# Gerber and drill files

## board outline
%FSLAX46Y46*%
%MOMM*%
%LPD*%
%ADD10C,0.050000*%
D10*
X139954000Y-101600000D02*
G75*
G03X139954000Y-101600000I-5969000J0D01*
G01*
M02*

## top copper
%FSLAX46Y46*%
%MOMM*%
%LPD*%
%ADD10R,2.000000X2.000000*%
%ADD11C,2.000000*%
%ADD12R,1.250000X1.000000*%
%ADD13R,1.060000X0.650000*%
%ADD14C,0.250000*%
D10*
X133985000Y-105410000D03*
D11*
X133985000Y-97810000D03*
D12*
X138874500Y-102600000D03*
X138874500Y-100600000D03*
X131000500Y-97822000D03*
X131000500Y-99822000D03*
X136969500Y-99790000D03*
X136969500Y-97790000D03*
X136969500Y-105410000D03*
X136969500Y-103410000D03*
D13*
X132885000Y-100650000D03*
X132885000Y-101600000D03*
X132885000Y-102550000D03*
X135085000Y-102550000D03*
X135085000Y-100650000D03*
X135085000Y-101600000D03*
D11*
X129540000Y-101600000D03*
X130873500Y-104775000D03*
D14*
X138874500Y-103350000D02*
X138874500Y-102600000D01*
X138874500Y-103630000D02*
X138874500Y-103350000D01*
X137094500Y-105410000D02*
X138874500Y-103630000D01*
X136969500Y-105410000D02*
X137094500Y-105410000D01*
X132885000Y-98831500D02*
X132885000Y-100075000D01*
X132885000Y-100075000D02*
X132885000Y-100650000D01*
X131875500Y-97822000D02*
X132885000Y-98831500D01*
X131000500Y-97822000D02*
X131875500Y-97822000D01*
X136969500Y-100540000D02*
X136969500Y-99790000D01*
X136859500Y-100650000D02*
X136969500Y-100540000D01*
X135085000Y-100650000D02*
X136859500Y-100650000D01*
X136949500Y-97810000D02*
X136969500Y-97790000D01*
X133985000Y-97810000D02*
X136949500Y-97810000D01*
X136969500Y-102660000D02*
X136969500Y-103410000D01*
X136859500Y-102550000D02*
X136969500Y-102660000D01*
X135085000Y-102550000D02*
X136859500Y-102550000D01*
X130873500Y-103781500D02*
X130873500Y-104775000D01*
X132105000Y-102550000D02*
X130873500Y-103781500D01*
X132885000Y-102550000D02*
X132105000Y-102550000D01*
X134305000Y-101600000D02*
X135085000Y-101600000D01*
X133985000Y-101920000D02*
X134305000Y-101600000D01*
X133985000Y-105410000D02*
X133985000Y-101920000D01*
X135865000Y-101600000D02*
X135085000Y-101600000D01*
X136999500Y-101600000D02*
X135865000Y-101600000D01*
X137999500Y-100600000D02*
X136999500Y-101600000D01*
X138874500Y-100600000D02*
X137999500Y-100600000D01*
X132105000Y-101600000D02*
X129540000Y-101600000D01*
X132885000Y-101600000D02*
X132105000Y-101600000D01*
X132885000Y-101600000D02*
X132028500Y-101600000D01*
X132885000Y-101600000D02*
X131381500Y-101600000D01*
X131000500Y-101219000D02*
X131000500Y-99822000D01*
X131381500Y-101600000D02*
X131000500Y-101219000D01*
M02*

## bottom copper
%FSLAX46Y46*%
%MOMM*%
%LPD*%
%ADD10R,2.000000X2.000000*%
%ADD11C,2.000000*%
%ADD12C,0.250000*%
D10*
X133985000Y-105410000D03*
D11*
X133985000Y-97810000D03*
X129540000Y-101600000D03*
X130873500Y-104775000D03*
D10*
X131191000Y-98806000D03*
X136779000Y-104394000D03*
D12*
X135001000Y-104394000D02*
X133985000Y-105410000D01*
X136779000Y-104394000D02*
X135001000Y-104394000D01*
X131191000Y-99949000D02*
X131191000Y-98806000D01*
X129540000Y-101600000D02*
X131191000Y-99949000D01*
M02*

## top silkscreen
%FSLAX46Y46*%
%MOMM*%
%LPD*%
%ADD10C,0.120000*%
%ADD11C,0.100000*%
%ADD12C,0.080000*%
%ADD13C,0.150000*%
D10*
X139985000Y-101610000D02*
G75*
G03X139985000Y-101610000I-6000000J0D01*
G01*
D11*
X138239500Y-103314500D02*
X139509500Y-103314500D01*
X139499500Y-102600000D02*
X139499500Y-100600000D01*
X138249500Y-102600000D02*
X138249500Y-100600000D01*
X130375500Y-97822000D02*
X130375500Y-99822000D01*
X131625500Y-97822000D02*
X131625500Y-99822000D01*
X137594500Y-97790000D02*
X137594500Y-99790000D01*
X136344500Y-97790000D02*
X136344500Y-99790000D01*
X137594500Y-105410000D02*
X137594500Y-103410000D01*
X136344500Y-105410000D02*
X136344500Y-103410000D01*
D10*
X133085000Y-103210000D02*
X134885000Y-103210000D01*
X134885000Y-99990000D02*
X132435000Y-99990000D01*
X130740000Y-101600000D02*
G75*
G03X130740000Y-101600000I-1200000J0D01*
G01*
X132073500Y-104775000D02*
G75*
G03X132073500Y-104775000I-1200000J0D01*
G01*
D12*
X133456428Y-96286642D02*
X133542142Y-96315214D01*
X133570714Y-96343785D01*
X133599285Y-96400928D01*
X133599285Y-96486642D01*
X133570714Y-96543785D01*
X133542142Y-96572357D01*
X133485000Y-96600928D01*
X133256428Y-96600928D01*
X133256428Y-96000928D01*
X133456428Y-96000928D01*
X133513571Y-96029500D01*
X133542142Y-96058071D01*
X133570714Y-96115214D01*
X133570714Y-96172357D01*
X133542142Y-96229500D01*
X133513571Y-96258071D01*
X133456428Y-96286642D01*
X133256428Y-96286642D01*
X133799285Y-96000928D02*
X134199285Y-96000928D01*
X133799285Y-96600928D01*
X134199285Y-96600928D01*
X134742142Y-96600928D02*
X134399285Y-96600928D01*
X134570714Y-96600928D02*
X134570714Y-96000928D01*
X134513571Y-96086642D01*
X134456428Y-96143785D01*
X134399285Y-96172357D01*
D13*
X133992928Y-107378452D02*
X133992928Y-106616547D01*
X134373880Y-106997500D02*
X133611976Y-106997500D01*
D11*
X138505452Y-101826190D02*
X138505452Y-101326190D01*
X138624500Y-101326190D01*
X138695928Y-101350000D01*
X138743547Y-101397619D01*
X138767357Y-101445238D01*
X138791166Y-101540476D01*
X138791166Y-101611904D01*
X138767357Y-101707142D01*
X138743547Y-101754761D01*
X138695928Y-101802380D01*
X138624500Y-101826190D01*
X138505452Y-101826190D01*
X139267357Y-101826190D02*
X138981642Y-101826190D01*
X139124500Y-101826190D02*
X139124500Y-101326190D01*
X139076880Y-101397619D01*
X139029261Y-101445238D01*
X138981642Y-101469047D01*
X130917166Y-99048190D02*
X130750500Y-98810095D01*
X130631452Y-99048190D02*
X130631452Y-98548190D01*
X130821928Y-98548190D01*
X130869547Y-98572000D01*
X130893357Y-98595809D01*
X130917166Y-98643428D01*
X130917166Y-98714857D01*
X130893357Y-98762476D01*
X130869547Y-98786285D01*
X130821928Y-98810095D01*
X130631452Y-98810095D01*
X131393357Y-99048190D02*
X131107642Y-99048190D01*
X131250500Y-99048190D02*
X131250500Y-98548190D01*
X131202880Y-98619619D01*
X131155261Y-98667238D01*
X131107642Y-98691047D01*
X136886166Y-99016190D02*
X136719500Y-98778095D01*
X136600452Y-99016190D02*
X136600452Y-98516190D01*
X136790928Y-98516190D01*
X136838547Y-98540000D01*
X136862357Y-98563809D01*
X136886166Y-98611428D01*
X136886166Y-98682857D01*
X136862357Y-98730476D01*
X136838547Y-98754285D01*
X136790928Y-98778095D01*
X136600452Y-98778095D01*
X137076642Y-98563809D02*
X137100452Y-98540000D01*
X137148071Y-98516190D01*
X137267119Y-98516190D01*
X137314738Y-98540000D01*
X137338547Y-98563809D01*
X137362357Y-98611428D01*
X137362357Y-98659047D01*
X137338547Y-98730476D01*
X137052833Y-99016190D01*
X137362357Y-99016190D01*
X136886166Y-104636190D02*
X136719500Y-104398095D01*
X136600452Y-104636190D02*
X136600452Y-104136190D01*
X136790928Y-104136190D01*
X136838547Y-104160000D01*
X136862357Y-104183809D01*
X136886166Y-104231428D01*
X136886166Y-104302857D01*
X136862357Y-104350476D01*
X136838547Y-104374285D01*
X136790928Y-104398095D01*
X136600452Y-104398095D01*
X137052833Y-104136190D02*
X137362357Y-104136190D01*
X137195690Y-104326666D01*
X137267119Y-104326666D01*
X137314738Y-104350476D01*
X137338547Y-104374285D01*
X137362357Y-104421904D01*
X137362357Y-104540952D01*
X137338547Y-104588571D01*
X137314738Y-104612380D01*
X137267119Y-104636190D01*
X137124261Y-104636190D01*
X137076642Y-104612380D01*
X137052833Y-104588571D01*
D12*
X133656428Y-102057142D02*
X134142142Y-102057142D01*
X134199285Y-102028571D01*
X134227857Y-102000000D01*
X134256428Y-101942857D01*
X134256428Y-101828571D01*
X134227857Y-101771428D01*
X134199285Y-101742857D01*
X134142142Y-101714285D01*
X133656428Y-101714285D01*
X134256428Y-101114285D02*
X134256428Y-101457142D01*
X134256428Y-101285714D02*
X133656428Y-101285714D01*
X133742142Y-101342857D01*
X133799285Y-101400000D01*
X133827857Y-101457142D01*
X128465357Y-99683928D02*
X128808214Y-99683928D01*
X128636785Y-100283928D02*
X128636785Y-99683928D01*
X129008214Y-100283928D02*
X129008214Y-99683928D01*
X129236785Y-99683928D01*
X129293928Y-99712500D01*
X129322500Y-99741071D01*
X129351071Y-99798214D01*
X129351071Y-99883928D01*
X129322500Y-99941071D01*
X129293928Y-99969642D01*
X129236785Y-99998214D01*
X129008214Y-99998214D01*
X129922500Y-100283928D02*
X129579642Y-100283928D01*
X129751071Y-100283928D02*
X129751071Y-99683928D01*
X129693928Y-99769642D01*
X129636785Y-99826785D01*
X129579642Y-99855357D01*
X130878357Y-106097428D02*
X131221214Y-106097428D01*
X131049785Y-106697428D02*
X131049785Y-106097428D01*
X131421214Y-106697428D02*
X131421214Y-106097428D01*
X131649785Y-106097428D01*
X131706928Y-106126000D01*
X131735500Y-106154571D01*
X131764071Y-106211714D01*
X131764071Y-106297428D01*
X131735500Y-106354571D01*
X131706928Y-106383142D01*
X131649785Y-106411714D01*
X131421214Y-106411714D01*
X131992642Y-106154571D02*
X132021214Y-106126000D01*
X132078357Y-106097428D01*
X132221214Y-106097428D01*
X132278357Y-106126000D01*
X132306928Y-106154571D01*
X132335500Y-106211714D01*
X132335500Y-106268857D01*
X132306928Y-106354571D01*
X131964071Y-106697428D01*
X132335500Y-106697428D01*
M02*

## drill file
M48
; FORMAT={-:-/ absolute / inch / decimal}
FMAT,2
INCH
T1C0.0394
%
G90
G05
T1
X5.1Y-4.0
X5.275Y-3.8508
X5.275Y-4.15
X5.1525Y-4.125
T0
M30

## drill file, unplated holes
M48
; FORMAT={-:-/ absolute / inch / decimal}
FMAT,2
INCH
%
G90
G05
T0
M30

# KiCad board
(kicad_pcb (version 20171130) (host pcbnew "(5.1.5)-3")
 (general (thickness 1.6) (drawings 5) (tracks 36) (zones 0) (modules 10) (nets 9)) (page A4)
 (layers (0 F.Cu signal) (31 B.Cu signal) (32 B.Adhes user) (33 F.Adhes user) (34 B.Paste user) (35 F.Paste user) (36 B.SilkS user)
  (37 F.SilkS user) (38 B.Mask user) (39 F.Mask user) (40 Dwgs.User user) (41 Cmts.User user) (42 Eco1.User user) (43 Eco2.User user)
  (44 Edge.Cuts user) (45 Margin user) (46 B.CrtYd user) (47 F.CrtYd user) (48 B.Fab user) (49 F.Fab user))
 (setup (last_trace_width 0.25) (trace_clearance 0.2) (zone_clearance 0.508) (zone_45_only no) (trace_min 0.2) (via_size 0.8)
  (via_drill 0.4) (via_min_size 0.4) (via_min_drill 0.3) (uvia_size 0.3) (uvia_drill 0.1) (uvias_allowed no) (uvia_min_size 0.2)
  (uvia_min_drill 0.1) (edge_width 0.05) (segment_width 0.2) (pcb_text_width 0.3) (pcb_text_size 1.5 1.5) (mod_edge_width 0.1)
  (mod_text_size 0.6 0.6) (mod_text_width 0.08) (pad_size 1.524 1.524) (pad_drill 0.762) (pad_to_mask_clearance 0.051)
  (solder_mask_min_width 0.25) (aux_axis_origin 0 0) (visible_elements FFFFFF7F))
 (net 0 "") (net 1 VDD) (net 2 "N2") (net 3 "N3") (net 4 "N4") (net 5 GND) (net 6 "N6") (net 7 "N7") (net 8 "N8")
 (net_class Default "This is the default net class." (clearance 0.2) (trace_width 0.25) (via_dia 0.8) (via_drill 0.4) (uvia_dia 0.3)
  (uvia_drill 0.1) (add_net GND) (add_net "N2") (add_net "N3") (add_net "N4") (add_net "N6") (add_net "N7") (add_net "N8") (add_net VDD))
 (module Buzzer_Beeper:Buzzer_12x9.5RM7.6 (layer F.Cu) (at 133.985 105.41 90)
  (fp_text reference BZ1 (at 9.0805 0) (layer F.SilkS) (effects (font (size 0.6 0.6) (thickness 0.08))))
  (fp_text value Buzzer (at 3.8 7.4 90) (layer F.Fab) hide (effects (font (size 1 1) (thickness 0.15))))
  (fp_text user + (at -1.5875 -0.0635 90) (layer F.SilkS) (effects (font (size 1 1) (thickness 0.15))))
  (fp_circle (center 3.8 0) (end 9.8 0) (layer F.SilkS) (width 0.12))
  (pad 1 thru_hole rect (at 0 0 90) (size 2 2) (drill 1) (layers *.Cu *.Mask) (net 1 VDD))
  (pad 2 thru_hole circle (at 7.6 0 90) (size 2 2) (drill 1) (layers *.Cu *.Mask) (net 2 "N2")))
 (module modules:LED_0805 (layer F.Cu) (at 138.8745 101.6 90)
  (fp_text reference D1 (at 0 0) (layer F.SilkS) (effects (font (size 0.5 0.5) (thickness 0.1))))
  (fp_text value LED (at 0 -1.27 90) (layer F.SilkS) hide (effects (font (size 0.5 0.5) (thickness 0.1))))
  (fp_line (start -1.7145 -0.635) (end -1.7145 0.635) (layer F.SilkS) (width 0.1))
  (fp_line (start -1 0.625) (end 1 0.625) (layer F.SilkS) (width 0.1))
  (fp_line (start -1 -0.625) (end 1 -0.625) (layer F.SilkS) (width 0.1))
  (pad 1 smd rect (at -1 0 90) (size 1 1.25) (layers F.Cu F.Paste F.Mask) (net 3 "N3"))
  (pad 2 smd rect (at 1 0 90) (size 1 1.25) (layers F.Cu F.Paste F.Mask) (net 1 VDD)))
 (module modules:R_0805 (layer F.Cu) (at 131.0005 98.822 270)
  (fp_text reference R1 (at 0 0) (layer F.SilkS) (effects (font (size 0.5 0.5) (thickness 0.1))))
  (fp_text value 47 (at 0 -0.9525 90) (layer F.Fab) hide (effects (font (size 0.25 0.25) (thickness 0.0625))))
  (fp_line (start -1 0.625) (end 1 0.625) (layer F.SilkS) (width 0.1))
  (fp_line (start -1 -0.625) (end 1 -0.625) (layer F.SilkS) (width 0.1))
  (pad 1 smd rect (at -1 0 270) (size 1 1.25) (layers F.Cu F.Paste F.Mask) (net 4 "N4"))
  (pad 2 smd rect (at 1 0 270) (size 1 1.25) (layers F.Cu F.Paste F.Mask) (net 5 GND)))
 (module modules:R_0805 (layer F.Cu) (at 136.9695 98.79 270)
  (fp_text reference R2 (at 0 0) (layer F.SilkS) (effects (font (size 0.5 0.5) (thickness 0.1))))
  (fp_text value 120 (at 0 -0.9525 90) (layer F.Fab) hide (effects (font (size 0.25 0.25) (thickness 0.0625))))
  (fp_line (start -1 -0.625) (end 1 -0.625) (layer F.SilkS) (width 0.1))
  (fp_line (start -1 0.625) (end 1 0.625) (layer F.SilkS) (width 0.1))
  (pad 2 smd rect (at 1 0 270) (size 1 1.25) (layers F.Cu F.Paste F.Mask) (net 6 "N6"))
  (pad 1 smd rect (at -1 0 270) (size 1 1.25) (layers F.Cu F.Paste F.Mask) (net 2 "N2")))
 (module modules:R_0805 (layer F.Cu) (at 136.9695 104.41 90)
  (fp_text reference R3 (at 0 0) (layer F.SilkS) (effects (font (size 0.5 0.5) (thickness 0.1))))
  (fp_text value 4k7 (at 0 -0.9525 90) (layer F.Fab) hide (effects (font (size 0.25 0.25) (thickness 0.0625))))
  (fp_line (start -1 0.625) (end 1 0.625) (layer F.SilkS) (width 0.1))
  (fp_line (start -1 -0.625) (end 1 -0.625) (layer F.SilkS) (width 0.1))
  (pad 1 smd rect (at -1 0 90) (size 1 1.25) (layers F.Cu F.Paste F.Mask) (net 3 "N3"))
  (pad 2 smd rect (at 1 0 90) (size 1 1.25) (layers F.Cu F.Paste F.Mask) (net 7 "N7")))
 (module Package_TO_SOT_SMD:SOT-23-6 (layer F.Cu) (at 133.985 101.6)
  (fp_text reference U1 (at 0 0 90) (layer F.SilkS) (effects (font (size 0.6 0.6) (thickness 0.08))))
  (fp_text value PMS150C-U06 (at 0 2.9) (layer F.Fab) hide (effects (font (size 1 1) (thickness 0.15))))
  (fp_line (start -0.9 1.61) (end 0.9 1.61) (layer F.SilkS) (width 0.12))
  (fp_line (start 0.9 -1.61) (end -1.55 -1.61) (layer F.SilkS) (width 0.12))
  (pad 1 smd rect (at -1.1 -0.95) (size 1.06 0.65) (layers F.Cu F.Paste F.Mask) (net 4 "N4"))
  (pad 2 smd rect (at -1.1 0) (size 1.06 0.65) (layers F.Cu F.Paste F.Mask) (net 5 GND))
  (pad 3 smd rect (at -1.1 0.95) (size 1.06 0.65) (layers F.Cu F.Paste F.Mask) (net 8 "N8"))
  (pad 4 smd rect (at 1.1 0.95) (size 1.06 0.65) (layers F.Cu F.Paste F.Mask) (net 7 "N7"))
  (pad 6 smd rect (at 1.1 -0.95) (size 1.06 0.65) (layers F.Cu F.Paste F.Mask) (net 6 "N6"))
  (pad 5 smd rect (at 1.1 0) (size 1.06 0.65) (layers F.Cu F.Paste F.Mask) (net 1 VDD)))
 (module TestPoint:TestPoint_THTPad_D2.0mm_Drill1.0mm (layer F.Cu) (at 129.54 101.6)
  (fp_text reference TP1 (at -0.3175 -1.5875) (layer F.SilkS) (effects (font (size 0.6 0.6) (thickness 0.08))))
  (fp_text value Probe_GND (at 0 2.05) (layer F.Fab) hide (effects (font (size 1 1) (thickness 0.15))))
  (fp_circle (center 0 0) (end 0 1.2) (layer F.SilkS) (width 0.12))
  (pad 1 thru_hole circle (at 0 0) (size 2 2) (drill 1) (layers *.Cu *.Mask) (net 5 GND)))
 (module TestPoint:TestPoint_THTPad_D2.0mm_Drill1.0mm (layer F.Cu) (at 130.8735 104.775)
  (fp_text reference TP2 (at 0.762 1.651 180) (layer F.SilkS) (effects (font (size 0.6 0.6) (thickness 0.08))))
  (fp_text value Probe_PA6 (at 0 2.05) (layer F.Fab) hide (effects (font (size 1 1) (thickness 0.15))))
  (fp_circle (center 0 0) (end 0 1.2) (layer F.SilkS) (width 0.12))
  (pad 1 thru_hole circle (at 0 0) (size 2 2) (drill 1) (layers *.Cu *.Mask) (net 8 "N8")))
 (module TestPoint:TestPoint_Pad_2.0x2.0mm (layer B.Cu) (at 131.191 98.806)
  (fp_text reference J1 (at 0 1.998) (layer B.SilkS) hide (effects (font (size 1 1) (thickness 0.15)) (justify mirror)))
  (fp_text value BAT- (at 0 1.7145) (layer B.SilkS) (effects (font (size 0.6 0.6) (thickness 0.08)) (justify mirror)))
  (pad 1 smd rect (at 0 0) (size 2 2) (layers B.Cu B.Mask) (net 5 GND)))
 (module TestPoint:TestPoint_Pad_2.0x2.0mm (layer B.Cu) (at 136.779 104.394)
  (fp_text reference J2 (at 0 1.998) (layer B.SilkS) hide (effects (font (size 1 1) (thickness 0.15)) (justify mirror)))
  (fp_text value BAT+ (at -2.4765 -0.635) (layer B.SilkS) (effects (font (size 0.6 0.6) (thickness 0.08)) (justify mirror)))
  (pad 1 smd rect (at 0 0) (size 2 2) (layers B.Cu B.Mask) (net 1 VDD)))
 (gr_circle (center 133.985 101.6) (end 139.954 101.6) (layer Edge.Cuts) (width 0.05))
 (segment (start 138.8745 103.35) (end 138.8745 102.6) (width 0.25) (layer F.Cu) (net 3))
 (segment (start 138.8745 103.63) (end 138.8745 103.35) (width 0.25) (layer F.Cu) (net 3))
 (segment (start 137.0945 105.41) (end 138.8745 103.63) (width 0.25) (layer F.Cu) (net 3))
 (segment (start 136.9695 105.41) (end 137.0945 105.41) (width 0.25) (layer F.Cu) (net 3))
 (segment (start 132.885 98.8315) (end 132.885 100.075) (width 0.25) (layer F.Cu) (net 4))
 (segment (start 132.885 100.075) (end 132.885 100.65) (width 0.25) (layer F.Cu) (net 4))
 (segment (start 131.8755 97.822) (end 132.885 98.8315) (width 0.25) (layer F.Cu) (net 4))
 (segment (start 131.0005 97.822) (end 131.8755 97.822) (width 0.25) (layer F.Cu) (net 4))
 (segment (start 136.9695 100.54) (end 136.9695 99.79) (width 0.25) (layer F.Cu) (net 6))
 (segment (start 136.8595 100.65) (end 136.9695 100.54) (width 0.25) (layer F.Cu) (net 6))
 (segment (start 135.085 100.65) (end 136.8595 100.65) (width 0.25) (layer F.Cu) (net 6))
 (segment (start 136.9495 97.81) (end 136.9695 97.79) (width 0.25) (layer F.Cu) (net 2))
 (segment (start 133.985 97.81) (end 136.9495 97.81) (width 0.25) (layer F.Cu) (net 2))
 (segment (start 136.9695 102.66) (end 136.9695 103.41) (width 0.25) (layer F.Cu) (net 7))
 (segment (start 136.8595 102.55) (end 136.9695 102.66) (width 0.25) (layer F.Cu) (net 7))
 (segment (start 135.085 102.55) (end 136.8595 102.55) (width 0.25) (layer F.Cu) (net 7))
 (segment (start 130.8735 103.7815) (end 130.8735 104.775) (width 0.25) (layer F.Cu) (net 8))
 (segment (start 132.105 102.55) (end 130.8735 103.7815) (width 0.25) (layer F.Cu) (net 8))
 (segment (start 132.885 102.55) (end 132.105 102.55) (width 0.25) (layer F.Cu) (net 8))
 (segment (start 134.305 101.6) (end 135.085 101.6) (width 0.25) (layer F.Cu) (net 1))
 (segment (start 133.985 101.92) (end 134.305 101.6) (width 0.25) (layer F.Cu) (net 1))
 (segment (start 133.985 105.41) (end 133.985 101.92) (width 0.25) (layer F.Cu) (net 1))
 (segment (start 135.865 101.6) (end 135.085 101.6) (width 0.25) (layer F.Cu) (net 1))
 (segment (start 136.9995 101.6) (end 135.865 101.6) (width 0.25) (layer F.Cu) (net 1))
 (segment (start 137.9995 100.6) (end 136.9995 101.6) (width 0.25) (layer F.Cu) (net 1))
 (segment (start 138.8745 100.6) (end 137.9995 100.6) (width 0.25) (layer F.Cu) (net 1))
 (segment (start 135.001 104.394) (end 133.985 105.41) (width 0.25) (layer B.Cu) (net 1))
 (segment (start 136.779 104.394) (end 135.001 104.394) (width 0.25) (layer B.Cu) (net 1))
 (segment (start 132.105 101.6) (end 129.54 101.6) (width 0.25) (layer F.Cu) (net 5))
 (segment (start 132.885 101.6) (end 132.105 101.6) (width 0.25) (layer F.Cu) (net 5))
 (segment (start 132.885 101.6) (end 132.0285 101.6) (width 0.25) (layer F.Cu) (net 5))
 (segment (start 132.885 101.6) (end 131.3815 101.6) (width 0.25) (layer F.Cu) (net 5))
 (segment (start 131.0005 101.219) (end 131.0005 99.822) (width 0.25) (layer F.Cu) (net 5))
 (segment (start 131.3815 101.6) (end 131.0005 101.219) (width 0.25) (layer F.Cu) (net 5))
 (segment (start 131.191 99.949) (end 131.191 98.806) (width 0.25) (layer B.Cu) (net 5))
 (segment (start 129.54 101.6) (end 131.191 99.949) (width 0.25) (layer B.Cu) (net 5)))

